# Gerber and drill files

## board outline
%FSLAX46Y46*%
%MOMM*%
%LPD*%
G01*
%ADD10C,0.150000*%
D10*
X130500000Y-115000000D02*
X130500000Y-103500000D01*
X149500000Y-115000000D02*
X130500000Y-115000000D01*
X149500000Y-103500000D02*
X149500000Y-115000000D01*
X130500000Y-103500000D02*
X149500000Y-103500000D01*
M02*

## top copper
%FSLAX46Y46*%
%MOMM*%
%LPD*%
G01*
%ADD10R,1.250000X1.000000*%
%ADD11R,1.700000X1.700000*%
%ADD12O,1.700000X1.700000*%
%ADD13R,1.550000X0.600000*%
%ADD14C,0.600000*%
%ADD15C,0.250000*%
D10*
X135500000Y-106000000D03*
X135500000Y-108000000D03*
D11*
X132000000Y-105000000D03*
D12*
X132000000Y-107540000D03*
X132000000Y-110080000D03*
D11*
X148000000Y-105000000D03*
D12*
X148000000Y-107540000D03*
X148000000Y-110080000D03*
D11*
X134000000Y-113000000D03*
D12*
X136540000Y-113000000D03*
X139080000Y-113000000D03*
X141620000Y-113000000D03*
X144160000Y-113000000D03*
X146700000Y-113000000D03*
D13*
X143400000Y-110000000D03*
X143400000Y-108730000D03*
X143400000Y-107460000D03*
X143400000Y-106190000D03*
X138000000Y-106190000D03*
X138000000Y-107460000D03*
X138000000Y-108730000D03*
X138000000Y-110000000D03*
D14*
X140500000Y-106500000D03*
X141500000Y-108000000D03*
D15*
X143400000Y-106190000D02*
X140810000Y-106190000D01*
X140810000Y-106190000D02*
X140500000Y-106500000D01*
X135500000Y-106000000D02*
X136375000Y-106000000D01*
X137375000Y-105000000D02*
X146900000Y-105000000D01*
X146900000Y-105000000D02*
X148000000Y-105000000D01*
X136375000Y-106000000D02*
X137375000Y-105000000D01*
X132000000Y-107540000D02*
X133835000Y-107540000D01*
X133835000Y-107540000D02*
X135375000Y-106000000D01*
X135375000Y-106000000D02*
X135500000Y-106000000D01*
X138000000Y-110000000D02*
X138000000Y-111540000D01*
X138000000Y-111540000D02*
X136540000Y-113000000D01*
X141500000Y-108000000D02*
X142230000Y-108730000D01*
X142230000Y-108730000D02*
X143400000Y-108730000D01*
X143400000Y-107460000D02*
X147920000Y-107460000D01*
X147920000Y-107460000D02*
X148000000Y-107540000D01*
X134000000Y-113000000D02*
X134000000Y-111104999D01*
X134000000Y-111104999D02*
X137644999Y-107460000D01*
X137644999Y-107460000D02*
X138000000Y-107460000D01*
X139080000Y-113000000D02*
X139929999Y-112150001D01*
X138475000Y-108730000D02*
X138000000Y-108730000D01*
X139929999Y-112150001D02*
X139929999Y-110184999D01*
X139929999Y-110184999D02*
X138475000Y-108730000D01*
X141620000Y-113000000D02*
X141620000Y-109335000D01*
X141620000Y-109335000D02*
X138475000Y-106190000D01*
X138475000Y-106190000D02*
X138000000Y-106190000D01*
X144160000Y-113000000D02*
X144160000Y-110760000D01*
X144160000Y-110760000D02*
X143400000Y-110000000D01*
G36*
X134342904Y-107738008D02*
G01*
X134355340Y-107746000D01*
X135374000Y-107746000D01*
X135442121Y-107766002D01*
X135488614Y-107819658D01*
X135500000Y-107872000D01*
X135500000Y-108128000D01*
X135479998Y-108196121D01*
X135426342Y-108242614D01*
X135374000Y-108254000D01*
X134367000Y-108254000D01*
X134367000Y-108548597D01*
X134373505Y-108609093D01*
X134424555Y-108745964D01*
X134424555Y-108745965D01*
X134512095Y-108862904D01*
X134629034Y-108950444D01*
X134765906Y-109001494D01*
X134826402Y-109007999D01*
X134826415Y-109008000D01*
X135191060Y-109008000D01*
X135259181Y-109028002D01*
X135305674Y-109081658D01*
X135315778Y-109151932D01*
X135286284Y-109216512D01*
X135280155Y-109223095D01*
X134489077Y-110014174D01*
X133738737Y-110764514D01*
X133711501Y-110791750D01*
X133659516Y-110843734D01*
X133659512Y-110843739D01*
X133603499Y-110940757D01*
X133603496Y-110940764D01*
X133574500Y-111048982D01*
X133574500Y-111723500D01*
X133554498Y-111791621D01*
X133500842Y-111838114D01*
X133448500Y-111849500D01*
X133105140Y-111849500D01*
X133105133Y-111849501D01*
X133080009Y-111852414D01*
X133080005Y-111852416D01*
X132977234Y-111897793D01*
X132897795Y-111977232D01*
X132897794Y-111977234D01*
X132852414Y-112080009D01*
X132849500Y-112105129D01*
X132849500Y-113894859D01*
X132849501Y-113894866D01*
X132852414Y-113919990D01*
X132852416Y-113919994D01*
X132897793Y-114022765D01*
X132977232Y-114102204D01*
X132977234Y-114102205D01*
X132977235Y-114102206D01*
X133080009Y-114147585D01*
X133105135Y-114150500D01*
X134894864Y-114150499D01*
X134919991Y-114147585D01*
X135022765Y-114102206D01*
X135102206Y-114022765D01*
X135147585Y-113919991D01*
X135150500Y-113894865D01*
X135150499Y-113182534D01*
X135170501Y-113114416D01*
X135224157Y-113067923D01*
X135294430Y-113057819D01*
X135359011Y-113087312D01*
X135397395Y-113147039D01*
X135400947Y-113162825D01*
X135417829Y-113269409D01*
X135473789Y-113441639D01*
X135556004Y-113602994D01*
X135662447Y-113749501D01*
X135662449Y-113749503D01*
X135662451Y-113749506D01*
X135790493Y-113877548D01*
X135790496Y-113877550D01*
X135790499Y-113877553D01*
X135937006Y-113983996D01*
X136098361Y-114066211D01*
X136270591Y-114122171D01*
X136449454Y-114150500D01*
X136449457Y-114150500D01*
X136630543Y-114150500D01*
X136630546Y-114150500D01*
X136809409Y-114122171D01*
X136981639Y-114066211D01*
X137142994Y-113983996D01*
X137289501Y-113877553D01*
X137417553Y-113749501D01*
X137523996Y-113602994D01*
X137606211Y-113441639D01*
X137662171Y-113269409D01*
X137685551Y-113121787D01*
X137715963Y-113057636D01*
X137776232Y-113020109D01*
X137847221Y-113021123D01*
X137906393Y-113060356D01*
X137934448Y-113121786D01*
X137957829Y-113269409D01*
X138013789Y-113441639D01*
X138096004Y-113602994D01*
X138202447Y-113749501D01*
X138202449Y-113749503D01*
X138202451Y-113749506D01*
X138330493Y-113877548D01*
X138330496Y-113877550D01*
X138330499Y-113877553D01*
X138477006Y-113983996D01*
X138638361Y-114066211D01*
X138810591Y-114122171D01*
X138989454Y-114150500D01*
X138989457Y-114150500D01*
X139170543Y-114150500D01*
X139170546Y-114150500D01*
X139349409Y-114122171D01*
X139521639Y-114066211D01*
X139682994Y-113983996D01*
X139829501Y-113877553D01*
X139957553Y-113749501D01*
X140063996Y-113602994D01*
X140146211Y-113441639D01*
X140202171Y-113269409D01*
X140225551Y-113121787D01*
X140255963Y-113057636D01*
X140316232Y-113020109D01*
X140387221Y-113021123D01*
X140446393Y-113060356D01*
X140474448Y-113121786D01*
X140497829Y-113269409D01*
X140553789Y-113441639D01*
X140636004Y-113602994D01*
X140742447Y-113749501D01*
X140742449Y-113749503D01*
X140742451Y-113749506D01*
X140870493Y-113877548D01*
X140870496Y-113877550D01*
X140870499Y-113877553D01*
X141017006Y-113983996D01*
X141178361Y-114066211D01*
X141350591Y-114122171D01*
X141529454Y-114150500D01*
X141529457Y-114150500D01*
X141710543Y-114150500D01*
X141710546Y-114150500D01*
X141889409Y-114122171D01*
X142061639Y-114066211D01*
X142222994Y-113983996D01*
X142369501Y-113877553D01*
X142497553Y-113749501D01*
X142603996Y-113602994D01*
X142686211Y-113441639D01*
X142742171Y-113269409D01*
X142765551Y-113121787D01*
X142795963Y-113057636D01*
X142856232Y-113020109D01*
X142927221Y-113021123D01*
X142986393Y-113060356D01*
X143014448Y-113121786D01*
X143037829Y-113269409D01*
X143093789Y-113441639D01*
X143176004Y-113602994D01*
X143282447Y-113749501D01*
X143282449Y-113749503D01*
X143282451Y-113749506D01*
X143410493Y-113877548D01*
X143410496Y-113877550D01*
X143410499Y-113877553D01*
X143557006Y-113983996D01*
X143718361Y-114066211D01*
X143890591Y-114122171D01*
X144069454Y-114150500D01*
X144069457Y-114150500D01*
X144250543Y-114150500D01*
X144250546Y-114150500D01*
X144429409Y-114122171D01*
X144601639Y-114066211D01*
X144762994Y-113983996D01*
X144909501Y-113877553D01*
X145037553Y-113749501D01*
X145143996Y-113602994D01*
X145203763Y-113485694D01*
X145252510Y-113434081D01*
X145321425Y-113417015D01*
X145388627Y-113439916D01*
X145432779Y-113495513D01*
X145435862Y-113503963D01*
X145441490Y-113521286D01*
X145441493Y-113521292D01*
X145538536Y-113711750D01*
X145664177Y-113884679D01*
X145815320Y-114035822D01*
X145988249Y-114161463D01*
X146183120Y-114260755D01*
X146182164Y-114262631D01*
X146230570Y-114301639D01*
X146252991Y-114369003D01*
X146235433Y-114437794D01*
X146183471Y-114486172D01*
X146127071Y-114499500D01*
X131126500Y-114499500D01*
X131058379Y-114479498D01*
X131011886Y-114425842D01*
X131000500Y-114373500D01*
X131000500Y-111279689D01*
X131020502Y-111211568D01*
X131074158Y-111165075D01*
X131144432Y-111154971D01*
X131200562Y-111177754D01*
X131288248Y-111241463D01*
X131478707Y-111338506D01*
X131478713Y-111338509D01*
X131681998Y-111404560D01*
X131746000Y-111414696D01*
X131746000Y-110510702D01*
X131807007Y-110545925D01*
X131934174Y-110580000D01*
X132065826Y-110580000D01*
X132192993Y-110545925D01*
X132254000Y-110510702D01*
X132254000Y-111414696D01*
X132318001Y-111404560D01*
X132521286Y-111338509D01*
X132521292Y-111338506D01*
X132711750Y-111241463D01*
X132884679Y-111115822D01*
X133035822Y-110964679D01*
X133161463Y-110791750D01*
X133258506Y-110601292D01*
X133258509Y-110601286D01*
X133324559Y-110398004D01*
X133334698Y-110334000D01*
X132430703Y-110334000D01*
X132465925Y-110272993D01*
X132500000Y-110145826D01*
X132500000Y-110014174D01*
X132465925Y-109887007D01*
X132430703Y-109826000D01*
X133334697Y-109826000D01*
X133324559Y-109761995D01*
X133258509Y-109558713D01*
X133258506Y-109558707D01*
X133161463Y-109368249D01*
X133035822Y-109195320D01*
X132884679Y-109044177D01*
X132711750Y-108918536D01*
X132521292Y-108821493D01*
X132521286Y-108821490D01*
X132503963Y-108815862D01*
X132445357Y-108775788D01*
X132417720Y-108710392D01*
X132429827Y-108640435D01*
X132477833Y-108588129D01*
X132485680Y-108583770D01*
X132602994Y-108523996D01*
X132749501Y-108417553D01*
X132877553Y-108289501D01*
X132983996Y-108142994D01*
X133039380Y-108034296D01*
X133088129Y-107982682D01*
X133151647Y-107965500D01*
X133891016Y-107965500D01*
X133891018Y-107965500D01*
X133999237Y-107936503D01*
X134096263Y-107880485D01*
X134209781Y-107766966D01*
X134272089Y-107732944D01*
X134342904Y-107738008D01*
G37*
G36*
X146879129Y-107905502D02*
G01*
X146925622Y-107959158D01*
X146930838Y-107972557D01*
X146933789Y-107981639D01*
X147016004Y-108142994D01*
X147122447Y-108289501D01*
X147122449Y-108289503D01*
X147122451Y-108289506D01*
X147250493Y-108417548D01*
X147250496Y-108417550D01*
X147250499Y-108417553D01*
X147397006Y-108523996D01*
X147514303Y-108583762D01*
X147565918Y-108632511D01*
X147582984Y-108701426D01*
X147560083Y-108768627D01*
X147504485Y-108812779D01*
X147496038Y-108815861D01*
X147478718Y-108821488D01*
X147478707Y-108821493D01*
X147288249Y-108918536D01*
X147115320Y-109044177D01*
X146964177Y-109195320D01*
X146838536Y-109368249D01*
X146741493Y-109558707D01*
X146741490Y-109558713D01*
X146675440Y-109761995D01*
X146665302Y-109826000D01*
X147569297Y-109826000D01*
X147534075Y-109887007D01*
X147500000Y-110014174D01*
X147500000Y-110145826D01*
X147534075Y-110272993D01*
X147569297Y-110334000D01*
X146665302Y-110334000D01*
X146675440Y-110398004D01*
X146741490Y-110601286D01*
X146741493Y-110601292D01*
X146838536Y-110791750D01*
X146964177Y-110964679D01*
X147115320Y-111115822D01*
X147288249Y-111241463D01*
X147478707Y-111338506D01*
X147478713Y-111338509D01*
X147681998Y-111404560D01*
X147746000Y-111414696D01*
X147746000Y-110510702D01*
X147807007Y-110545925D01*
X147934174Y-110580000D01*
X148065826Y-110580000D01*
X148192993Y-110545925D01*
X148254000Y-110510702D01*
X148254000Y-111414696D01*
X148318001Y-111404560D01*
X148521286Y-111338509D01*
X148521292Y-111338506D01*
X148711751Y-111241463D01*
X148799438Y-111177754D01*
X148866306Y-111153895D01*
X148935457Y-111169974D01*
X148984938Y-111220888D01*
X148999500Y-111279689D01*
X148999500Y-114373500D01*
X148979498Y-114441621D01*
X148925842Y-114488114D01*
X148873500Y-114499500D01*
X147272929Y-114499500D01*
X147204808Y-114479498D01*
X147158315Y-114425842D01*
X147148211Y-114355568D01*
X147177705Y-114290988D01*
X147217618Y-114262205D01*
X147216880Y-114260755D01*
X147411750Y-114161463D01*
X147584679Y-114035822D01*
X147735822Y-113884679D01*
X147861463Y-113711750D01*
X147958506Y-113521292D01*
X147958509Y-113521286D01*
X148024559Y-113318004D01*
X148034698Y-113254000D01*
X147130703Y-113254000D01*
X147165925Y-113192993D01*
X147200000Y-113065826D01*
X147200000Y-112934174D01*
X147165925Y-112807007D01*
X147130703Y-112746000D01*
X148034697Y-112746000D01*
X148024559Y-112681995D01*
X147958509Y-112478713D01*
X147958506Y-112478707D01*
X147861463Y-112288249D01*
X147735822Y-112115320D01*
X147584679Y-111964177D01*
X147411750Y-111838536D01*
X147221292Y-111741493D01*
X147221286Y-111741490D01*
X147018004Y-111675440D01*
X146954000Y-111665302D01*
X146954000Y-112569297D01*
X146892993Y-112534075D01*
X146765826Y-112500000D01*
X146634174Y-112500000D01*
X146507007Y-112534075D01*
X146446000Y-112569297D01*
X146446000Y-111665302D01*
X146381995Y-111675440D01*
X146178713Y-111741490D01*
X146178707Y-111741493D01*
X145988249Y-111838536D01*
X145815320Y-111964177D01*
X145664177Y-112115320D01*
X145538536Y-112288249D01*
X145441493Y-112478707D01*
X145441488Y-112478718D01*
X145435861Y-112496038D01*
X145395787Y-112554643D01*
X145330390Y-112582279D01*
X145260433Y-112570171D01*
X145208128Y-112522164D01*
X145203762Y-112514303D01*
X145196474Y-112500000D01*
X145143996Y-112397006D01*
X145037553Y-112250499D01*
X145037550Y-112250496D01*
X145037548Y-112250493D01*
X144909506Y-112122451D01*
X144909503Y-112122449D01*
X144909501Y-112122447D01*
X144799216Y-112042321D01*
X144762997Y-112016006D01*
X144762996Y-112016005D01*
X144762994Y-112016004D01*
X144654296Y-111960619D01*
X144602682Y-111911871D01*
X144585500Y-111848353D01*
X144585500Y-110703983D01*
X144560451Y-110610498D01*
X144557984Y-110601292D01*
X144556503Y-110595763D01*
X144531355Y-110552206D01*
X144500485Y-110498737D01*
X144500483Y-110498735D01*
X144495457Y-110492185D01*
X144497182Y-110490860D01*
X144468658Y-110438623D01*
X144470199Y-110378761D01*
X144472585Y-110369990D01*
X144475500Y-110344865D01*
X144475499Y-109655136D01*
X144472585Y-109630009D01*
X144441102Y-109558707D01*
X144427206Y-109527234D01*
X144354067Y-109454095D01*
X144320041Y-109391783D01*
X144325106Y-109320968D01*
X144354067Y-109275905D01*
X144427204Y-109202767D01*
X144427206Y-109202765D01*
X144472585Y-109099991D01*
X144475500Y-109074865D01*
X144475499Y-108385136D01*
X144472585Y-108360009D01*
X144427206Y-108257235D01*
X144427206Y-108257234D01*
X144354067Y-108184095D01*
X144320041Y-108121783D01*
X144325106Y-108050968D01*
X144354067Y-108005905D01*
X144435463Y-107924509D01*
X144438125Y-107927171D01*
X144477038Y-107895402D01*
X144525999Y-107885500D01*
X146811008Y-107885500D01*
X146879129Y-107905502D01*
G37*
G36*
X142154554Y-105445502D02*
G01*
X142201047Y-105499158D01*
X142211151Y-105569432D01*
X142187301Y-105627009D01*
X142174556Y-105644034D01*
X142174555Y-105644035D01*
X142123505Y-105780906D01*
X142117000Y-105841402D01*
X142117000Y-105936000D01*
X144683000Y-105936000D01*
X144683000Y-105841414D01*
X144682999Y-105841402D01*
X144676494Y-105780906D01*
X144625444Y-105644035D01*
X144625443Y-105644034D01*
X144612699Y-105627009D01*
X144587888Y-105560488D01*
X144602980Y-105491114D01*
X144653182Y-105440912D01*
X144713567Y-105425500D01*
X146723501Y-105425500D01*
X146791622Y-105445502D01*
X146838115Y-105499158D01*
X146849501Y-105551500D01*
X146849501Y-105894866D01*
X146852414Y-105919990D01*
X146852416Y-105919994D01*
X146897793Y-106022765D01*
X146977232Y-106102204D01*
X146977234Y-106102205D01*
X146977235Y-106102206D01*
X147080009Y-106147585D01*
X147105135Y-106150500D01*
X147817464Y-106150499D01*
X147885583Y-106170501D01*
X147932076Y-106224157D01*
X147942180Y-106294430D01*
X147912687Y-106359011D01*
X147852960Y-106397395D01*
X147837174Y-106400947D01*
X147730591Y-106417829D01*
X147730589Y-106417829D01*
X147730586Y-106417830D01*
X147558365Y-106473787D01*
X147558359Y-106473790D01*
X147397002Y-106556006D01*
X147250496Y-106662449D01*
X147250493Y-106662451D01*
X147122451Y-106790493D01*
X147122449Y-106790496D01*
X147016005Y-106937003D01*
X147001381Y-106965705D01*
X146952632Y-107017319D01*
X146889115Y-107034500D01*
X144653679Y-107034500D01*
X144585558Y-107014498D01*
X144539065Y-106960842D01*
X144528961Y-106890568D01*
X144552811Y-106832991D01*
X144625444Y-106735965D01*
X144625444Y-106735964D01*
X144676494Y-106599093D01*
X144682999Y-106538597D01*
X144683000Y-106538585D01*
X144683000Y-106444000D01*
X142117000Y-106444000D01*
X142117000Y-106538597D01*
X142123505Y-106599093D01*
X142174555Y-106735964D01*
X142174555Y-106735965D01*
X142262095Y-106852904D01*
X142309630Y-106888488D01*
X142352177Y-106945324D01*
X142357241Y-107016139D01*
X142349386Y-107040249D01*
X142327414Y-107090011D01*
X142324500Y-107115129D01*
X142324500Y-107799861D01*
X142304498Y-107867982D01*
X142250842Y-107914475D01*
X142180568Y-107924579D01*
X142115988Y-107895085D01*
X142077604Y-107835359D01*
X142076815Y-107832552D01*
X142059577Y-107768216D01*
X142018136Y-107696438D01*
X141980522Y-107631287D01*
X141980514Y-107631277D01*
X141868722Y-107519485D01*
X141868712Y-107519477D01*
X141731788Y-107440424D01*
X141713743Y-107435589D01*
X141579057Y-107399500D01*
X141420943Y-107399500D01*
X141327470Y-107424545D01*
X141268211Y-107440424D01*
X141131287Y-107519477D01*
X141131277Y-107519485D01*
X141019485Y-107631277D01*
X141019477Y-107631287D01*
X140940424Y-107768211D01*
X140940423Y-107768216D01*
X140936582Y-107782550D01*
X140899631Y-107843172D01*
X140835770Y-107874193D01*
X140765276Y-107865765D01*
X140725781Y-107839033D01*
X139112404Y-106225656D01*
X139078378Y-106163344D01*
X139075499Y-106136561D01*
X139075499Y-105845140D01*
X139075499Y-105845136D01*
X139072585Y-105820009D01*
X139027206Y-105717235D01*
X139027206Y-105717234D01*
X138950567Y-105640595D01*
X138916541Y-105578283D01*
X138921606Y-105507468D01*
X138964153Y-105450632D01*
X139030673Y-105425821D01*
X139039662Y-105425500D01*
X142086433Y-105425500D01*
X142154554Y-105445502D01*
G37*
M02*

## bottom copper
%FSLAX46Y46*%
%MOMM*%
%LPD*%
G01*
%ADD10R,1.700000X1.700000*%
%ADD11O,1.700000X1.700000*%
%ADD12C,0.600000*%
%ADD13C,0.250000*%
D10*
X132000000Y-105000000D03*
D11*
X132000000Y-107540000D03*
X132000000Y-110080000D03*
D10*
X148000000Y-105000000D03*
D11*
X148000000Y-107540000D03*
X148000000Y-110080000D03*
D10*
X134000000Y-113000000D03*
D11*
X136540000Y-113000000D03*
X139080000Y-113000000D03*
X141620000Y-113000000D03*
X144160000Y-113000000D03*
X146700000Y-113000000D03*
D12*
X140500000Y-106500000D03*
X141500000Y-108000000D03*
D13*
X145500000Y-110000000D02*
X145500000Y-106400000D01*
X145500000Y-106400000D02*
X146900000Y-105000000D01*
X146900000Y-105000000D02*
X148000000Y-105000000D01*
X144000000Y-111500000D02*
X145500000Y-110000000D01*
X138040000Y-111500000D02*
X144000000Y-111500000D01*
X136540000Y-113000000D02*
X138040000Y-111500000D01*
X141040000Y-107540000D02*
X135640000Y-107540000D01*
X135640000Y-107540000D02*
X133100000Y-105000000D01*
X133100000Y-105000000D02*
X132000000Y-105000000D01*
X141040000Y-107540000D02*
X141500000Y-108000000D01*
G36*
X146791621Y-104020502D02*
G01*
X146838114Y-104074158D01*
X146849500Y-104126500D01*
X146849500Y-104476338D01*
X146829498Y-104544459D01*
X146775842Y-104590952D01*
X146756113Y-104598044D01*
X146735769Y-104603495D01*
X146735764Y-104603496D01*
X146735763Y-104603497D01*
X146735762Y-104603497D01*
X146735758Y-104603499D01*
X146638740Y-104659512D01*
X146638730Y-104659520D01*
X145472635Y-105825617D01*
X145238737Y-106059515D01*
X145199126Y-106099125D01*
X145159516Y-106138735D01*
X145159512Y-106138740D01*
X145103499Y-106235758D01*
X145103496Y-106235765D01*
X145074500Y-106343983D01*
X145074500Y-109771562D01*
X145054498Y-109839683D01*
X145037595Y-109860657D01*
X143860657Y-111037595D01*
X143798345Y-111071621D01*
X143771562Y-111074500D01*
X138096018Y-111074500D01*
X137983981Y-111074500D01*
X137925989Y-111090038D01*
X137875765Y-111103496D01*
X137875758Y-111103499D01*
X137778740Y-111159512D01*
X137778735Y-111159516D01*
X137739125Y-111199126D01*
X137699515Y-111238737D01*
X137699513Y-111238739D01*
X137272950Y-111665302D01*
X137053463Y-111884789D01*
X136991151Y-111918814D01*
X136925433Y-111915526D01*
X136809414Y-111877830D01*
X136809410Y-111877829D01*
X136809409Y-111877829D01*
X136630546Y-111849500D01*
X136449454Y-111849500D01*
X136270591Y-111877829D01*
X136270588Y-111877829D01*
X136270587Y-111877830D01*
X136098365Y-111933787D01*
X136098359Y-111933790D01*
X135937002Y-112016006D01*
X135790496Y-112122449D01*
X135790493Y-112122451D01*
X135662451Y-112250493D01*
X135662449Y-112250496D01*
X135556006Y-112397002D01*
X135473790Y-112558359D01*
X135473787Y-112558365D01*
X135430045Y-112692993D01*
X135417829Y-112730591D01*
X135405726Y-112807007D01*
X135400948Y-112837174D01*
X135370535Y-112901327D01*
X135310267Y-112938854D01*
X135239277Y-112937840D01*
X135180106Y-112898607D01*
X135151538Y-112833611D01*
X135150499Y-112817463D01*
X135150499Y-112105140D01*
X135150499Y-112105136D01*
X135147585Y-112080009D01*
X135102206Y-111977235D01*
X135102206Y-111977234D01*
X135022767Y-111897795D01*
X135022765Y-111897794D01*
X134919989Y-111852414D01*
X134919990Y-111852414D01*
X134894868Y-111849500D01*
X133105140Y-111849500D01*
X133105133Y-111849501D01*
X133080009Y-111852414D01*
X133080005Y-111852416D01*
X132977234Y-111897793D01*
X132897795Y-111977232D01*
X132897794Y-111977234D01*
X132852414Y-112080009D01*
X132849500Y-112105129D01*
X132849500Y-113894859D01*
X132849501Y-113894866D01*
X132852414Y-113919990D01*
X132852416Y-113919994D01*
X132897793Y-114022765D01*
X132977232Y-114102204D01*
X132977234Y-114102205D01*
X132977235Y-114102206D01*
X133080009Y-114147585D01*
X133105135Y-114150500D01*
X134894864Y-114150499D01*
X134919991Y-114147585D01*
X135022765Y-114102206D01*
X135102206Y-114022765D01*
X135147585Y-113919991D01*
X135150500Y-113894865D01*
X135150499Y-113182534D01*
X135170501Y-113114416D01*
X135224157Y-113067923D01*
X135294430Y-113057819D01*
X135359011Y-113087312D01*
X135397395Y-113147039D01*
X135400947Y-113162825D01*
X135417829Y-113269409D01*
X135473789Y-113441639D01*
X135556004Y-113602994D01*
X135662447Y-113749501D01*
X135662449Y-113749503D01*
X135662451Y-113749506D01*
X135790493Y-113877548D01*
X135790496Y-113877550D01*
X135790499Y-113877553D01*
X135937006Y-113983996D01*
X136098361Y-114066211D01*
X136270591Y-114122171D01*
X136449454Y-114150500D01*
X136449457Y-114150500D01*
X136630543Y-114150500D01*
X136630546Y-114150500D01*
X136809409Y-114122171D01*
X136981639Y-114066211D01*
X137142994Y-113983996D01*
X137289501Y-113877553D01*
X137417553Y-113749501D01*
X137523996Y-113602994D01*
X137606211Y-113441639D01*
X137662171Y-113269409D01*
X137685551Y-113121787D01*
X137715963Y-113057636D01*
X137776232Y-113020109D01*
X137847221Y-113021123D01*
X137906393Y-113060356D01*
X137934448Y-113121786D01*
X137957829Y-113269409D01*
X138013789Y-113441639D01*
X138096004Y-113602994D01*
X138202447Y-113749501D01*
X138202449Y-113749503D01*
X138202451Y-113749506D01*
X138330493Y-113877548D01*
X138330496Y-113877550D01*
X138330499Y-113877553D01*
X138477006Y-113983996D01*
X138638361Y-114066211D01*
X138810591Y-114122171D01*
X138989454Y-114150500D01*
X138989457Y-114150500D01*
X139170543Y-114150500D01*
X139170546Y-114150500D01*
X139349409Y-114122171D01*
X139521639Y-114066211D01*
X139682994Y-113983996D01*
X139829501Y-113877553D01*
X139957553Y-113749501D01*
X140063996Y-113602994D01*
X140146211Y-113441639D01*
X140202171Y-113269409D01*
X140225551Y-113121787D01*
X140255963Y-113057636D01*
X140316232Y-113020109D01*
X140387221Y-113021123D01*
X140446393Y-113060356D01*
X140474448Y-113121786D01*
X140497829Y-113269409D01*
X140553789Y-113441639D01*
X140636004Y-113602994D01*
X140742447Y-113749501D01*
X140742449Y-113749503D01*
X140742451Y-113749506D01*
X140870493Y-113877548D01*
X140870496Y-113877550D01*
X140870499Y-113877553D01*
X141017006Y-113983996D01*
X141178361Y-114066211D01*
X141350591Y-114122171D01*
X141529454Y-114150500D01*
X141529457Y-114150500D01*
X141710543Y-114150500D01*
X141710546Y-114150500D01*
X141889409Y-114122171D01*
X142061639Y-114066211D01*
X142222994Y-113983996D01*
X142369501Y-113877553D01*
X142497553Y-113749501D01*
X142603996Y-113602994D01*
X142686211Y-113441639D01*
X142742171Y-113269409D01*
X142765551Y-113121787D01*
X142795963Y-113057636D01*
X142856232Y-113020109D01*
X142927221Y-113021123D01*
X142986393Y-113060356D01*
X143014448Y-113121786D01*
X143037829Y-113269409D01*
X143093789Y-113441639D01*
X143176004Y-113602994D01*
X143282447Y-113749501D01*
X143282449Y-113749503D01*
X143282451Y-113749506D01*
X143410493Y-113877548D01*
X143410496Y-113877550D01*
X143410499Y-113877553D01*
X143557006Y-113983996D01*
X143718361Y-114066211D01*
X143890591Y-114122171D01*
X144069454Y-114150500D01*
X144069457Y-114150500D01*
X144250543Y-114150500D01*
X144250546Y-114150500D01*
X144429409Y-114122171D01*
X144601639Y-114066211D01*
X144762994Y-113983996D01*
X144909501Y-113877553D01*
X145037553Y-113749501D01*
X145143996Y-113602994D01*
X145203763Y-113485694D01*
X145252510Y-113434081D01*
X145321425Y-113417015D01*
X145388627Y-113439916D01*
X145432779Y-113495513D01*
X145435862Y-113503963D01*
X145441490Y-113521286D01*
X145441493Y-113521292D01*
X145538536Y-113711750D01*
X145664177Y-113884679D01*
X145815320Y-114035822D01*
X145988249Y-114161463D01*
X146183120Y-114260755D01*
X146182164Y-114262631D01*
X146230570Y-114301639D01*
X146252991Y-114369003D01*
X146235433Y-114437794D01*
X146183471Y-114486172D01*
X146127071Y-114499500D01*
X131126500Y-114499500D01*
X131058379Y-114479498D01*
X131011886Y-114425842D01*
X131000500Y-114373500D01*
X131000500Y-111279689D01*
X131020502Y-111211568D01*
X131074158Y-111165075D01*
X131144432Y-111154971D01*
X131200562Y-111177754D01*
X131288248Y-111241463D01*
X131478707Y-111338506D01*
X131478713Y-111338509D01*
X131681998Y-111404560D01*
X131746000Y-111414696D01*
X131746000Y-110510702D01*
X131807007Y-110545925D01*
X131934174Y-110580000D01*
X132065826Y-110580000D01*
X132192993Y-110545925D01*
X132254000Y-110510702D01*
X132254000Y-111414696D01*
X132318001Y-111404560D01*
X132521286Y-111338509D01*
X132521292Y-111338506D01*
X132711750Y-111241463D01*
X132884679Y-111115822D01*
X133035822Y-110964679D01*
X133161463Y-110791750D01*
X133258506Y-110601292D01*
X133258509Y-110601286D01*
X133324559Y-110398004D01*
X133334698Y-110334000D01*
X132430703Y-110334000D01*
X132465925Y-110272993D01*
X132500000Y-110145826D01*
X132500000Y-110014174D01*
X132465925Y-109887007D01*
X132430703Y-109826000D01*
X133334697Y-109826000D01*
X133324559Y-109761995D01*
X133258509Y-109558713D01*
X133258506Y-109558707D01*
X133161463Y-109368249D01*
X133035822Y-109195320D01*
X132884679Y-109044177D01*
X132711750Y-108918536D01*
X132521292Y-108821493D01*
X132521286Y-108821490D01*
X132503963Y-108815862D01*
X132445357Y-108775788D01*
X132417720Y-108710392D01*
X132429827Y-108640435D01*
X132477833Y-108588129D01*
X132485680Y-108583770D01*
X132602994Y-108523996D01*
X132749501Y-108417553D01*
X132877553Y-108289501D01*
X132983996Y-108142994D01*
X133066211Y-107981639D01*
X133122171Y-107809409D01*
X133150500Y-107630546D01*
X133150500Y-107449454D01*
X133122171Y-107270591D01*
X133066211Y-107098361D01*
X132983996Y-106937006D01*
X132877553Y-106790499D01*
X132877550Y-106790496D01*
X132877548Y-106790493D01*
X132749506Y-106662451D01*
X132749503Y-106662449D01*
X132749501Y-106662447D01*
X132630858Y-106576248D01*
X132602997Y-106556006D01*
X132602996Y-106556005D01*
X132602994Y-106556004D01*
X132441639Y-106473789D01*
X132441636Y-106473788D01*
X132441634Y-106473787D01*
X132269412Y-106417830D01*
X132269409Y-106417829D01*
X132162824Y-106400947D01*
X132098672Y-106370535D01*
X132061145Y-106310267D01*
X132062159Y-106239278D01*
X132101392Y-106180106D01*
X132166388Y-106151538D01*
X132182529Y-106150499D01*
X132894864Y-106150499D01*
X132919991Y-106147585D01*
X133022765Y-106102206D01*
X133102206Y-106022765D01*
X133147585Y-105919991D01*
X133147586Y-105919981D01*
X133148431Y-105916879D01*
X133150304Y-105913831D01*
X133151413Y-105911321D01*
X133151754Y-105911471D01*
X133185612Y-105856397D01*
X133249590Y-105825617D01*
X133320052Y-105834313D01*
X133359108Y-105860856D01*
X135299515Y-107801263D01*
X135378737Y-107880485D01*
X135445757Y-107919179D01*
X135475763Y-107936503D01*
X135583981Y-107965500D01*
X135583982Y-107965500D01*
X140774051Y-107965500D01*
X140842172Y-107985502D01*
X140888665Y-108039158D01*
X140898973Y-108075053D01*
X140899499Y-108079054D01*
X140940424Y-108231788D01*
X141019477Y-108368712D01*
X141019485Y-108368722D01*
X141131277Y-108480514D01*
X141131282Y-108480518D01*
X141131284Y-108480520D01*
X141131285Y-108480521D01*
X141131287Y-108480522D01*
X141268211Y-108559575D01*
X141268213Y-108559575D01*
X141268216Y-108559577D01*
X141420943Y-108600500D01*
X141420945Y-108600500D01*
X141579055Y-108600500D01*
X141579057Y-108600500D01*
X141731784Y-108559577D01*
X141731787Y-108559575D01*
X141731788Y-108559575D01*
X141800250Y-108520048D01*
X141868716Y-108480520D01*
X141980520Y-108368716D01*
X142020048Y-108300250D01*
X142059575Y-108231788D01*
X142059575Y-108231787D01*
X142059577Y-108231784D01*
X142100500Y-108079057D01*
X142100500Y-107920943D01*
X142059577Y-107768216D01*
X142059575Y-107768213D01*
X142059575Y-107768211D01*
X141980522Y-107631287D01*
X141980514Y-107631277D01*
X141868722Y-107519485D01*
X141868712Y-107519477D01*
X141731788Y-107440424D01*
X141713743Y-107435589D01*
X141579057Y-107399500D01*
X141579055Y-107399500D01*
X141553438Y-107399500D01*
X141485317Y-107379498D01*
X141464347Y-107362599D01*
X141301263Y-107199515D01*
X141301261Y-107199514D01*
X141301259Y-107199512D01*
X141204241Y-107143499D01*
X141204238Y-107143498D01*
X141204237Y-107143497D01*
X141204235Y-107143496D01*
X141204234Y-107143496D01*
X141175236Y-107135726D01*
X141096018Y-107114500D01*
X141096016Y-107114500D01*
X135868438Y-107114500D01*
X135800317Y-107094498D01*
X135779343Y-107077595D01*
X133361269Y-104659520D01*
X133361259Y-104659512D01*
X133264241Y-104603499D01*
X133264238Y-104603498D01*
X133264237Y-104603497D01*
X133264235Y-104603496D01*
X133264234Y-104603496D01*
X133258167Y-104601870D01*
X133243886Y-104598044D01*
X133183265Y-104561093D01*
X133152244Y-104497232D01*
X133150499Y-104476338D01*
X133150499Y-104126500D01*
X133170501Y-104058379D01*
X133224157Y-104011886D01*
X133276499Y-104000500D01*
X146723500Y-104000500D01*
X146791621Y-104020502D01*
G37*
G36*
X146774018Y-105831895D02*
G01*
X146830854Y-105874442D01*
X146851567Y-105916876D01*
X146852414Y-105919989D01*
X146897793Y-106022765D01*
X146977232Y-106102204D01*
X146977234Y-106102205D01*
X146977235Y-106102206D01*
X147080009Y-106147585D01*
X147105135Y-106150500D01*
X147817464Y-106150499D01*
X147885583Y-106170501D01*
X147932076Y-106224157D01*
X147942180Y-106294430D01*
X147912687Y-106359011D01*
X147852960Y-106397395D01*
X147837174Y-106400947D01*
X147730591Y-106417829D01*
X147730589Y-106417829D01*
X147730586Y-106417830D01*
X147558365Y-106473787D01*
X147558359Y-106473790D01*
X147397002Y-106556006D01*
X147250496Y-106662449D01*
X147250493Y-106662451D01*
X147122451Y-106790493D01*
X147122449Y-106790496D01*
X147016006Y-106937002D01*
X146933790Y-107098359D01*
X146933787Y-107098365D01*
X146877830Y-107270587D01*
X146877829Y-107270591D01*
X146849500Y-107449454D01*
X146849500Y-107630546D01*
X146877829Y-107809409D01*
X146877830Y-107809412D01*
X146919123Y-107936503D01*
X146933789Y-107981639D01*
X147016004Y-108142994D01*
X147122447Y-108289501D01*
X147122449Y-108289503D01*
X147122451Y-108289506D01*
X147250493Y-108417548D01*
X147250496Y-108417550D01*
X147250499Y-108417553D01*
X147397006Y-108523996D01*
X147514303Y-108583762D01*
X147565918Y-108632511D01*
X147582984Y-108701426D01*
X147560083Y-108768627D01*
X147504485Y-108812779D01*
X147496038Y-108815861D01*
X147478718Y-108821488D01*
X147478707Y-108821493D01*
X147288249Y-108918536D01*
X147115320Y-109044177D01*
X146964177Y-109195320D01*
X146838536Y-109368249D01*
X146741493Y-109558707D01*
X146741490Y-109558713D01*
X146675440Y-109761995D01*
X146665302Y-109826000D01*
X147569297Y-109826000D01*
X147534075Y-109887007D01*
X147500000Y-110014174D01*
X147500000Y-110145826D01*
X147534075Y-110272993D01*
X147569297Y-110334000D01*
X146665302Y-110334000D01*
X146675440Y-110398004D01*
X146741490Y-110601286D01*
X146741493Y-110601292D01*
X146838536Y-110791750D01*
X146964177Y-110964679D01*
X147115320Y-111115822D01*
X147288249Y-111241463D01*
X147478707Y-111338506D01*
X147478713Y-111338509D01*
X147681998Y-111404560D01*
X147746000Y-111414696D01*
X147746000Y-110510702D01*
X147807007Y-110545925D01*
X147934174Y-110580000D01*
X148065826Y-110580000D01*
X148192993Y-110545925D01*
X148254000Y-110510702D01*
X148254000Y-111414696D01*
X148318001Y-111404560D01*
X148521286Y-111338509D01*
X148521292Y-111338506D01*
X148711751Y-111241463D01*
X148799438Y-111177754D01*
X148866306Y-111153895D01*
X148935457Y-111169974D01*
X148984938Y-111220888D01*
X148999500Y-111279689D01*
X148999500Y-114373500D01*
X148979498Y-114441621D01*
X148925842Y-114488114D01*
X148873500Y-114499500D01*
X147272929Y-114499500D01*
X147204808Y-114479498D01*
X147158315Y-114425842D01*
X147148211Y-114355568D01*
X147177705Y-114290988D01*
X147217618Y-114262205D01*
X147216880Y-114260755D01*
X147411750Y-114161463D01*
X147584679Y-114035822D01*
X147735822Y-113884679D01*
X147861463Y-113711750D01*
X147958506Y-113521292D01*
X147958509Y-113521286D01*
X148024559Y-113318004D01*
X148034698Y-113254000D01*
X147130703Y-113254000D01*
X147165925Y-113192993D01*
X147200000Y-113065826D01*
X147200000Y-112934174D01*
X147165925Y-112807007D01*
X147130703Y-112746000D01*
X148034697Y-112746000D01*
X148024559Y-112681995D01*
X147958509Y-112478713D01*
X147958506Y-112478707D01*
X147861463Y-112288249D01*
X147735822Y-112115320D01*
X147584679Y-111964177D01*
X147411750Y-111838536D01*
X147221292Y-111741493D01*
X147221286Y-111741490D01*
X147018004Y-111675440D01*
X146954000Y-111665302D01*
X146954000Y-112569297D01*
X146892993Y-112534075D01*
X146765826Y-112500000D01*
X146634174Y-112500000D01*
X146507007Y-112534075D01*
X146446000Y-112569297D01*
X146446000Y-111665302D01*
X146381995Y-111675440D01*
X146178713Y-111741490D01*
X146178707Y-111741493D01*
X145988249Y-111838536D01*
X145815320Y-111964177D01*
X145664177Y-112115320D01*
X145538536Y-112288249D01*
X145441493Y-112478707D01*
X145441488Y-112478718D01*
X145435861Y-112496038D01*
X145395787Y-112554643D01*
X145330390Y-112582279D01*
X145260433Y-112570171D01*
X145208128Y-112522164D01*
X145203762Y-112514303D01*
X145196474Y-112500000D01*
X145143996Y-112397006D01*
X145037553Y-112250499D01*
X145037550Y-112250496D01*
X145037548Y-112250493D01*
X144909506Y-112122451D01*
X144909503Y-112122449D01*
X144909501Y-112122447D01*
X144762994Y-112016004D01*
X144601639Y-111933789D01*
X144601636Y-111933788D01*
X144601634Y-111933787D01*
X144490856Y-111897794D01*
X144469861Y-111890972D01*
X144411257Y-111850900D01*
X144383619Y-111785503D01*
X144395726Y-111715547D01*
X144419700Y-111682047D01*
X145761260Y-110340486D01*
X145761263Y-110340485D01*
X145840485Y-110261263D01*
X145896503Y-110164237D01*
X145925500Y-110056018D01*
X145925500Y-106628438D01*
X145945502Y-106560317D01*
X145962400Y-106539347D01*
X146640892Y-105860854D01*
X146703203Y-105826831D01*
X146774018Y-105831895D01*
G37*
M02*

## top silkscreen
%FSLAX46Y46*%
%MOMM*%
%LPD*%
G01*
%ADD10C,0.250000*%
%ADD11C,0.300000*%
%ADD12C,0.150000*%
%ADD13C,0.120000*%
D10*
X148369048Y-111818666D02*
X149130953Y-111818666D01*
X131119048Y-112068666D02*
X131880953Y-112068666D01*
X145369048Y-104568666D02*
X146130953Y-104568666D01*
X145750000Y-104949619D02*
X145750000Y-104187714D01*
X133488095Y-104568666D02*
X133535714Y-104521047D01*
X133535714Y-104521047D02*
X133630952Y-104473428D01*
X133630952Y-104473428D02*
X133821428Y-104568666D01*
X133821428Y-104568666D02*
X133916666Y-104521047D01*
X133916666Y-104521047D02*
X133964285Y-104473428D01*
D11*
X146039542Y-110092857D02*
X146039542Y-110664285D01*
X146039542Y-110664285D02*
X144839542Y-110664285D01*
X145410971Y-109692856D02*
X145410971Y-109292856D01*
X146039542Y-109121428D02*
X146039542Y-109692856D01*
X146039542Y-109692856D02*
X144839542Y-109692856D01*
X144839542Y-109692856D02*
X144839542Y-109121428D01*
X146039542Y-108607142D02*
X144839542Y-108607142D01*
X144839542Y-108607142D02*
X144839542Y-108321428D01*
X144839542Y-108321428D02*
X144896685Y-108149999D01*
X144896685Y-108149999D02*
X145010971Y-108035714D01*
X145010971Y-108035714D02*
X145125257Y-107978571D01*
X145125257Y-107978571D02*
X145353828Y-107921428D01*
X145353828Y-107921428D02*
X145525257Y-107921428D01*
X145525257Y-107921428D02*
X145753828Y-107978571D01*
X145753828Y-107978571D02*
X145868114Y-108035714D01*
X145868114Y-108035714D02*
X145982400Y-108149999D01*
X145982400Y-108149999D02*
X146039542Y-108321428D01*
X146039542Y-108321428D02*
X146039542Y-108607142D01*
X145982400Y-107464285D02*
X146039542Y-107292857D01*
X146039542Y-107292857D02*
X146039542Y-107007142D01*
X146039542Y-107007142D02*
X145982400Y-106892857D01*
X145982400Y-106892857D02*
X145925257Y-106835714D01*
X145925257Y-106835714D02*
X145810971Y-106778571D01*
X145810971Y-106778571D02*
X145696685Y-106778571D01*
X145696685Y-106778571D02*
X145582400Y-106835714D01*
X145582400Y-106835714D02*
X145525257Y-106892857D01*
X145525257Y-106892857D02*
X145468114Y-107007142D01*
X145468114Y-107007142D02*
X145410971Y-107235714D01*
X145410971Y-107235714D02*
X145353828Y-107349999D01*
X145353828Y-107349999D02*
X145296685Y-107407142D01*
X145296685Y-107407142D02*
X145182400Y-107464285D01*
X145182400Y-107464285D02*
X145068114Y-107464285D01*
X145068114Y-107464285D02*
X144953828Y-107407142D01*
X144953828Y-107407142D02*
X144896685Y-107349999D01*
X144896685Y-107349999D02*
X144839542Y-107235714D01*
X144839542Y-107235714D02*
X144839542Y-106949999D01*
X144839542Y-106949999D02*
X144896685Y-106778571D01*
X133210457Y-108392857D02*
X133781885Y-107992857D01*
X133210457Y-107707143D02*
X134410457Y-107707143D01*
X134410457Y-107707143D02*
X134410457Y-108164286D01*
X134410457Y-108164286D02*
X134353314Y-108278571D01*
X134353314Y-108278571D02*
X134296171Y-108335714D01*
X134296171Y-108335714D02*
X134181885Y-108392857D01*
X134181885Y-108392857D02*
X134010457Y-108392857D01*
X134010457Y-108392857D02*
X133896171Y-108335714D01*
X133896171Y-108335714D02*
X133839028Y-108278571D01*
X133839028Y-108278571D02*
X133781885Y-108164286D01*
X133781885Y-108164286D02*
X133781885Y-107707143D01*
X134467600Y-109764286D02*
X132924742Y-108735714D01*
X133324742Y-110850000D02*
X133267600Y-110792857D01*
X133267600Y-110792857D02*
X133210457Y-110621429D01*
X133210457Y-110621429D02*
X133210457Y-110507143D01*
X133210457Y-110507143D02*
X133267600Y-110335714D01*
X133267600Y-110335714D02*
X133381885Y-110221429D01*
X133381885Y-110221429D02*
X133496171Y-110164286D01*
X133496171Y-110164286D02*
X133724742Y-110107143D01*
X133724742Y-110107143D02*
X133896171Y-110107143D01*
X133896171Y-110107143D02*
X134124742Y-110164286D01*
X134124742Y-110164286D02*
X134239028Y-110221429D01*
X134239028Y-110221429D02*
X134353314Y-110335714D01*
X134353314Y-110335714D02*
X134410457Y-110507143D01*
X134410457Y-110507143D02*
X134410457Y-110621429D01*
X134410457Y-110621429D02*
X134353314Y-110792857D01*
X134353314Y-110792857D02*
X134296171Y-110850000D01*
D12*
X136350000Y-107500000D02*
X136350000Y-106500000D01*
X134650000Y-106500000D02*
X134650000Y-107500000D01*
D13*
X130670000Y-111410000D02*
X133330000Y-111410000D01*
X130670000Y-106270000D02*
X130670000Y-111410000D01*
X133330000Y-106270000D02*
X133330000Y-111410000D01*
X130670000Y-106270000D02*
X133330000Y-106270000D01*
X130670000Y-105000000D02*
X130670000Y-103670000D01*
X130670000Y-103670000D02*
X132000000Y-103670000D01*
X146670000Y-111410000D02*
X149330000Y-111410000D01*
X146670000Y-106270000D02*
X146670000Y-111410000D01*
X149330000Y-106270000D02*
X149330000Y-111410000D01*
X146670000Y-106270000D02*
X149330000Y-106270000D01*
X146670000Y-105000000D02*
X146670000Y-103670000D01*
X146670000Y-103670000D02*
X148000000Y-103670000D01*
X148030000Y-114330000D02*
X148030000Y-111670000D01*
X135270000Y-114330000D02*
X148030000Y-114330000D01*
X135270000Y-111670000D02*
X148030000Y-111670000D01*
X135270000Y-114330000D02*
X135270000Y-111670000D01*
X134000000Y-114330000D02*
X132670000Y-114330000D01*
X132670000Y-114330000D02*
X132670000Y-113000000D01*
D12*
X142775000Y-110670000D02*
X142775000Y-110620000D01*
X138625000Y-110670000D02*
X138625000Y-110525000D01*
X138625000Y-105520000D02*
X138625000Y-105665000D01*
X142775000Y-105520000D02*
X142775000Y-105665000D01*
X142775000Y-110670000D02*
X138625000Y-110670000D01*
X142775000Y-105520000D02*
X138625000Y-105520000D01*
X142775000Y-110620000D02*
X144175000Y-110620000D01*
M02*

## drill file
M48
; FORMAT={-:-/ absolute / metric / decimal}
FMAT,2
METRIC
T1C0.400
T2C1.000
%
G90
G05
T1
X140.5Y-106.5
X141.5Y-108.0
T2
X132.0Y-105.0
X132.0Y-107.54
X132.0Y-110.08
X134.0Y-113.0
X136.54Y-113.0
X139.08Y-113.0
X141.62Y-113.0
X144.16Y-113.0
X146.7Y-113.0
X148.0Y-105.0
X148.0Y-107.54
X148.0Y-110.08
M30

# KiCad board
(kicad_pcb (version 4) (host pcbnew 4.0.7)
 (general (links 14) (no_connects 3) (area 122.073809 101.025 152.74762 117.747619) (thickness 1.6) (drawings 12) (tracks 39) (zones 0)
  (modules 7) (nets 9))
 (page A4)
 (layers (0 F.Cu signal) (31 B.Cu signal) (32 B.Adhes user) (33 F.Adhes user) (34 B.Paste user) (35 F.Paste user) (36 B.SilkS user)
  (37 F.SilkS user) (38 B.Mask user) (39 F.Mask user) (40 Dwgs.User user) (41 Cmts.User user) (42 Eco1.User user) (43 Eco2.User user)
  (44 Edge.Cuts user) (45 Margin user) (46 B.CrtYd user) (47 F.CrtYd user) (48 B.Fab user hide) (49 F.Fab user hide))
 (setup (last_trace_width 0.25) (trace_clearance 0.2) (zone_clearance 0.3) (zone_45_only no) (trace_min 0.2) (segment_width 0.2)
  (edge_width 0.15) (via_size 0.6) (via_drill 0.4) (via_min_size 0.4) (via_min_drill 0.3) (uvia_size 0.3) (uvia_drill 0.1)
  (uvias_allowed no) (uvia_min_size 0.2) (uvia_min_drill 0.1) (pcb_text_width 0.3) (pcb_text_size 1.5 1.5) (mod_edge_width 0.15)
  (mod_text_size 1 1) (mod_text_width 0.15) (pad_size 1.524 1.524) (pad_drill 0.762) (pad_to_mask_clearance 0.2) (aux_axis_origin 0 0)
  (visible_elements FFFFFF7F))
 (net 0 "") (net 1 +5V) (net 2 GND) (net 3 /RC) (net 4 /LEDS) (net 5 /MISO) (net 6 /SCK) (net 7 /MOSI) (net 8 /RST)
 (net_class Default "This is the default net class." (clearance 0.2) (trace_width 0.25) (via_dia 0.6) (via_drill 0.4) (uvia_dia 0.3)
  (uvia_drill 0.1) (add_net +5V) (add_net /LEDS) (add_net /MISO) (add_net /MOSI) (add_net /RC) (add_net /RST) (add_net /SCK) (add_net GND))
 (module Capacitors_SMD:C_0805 (layer F.Cu) (at 135.5 107 270)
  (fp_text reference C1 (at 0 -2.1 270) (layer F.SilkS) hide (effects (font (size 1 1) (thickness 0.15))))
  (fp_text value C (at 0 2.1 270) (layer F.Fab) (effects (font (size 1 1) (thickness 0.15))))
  (fp_line (start 0.5 -0.85) (end -0.5 -0.85) (layer F.SilkS) (width 0.15))
  (fp_line (start -0.5 0.85) (end 0.5 0.85) (layer F.SilkS) (width 0.15))
  (pad 1 smd rect (at -1 0 270) (size 1 1.25) (layers F.Cu F.Paste F.Mask) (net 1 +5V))
  (pad 2 smd rect (at 1 0 270) (size 1 1.25) (layers F.Cu F.Paste F.Mask) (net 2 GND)))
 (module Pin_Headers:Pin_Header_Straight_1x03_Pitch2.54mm (layer F.Cu) (at 132 105)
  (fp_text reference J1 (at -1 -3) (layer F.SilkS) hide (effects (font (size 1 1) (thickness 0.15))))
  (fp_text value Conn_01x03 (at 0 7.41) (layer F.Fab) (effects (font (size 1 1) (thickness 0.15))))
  (fp_line (start -1.33 6.41) (end 1.33 6.41) (layer F.SilkS) (width 0.12))
  (fp_line (start -1.33 1.27) (end -1.33 6.41) (layer F.SilkS) (width 0.12))
  (fp_line (start 1.33 1.27) (end 1.33 6.41) (layer F.SilkS) (width 0.12))
  (fp_line (start -1.33 1.27) (end 1.33 1.27) (layer F.SilkS) (width 0.12))
  (fp_line (start -1.33 0) (end -1.33 -1.33) (layer F.SilkS) (width 0.12))
  (fp_line (start -1.33 -1.33) (end 0 -1.33) (layer F.SilkS) (width 0.12))
  (pad 1 thru_hole rect (at 0 0) (size 1.7 1.7) (drill 1) (layers *.Cu *.Mask) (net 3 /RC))
  (pad 2 thru_hole oval (at 0 2.54) (size 1.7 1.7) (drill 1) (layers *.Cu *.Mask) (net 1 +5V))
  (pad 3 thru_hole oval (at 0 5.08) (size 1.7 1.7) (drill 1) (layers *.Cu *.Mask) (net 2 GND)))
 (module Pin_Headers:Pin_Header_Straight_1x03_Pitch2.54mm (layer F.Cu) (at 148 105)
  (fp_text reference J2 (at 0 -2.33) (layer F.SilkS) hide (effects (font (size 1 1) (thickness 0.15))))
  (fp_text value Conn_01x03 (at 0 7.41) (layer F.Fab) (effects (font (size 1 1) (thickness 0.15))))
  (fp_line (start -1.33 6.41) (end 1.33 6.41) (layer F.SilkS) (width 0.12))
  (fp_line (start -1.33 1.27) (end -1.33 6.41) (layer F.SilkS) (width 0.12))
  (fp_line (start 1.33 1.27) (end 1.33 6.41) (layer F.SilkS) (width 0.12))
  (fp_line (start -1.33 1.27) (end 1.33 1.27) (layer F.SilkS) (width 0.12))
  (fp_line (start -1.33 0) (end -1.33 -1.33) (layer F.SilkS) (width 0.12))
  (fp_line (start -1.33 -1.33) (end 0 -1.33) (layer F.SilkS) (width 0.12))
  (pad 1 thru_hole rect (at 0 0) (size 1.7 1.7) (drill 1) (layers *.Cu *.Mask) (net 1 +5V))
  (pad 2 thru_hole oval (at 0 2.54) (size 1.7 1.7) (drill 1) (layers *.Cu *.Mask) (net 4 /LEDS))
  (pad 3 thru_hole oval (at 0 5.08) (size 1.7 1.7) (drill 1) (layers *.Cu *.Mask) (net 2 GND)))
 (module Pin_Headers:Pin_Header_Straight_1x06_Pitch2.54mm (layer F.Cu) (at 134 113 90)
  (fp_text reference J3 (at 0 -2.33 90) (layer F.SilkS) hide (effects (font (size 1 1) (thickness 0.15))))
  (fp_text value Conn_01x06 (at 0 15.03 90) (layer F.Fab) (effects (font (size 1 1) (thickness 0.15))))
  (fp_line (start -1.33 14.03) (end 1.33 14.03) (layer F.SilkS) (width 0.12))
  (fp_line (start -1.33 1.27) (end -1.33 14.03) (layer F.SilkS) (width 0.12))
  (fp_line (start 1.33 1.27) (end 1.33 14.03) (layer F.SilkS) (width 0.12))
  (fp_line (start -1.33 1.27) (end 1.33 1.27) (layer F.SilkS) (width 0.12))
  (fp_line (start -1.33 0) (end -1.33 -1.33) (layer F.SilkS) (width 0.12))
  (fp_line (start -1.33 -1.33) (end 0 -1.33) (layer F.SilkS) (width 0.12))
  (pad 1 thru_hole rect (at 0 0 90) (size 1.7 1.7) (drill 1) (layers *.Cu *.Mask) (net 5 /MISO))
  (pad 2 thru_hole oval (at 0 2.54 90) (size 1.7 1.7) (drill 1) (layers *.Cu *.Mask) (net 1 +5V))
  (pad 3 thru_hole oval (at 0 5.08 90) (size 1.7 1.7) (drill 1) (layers *.Cu *.Mask) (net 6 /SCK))
  (pad 4 thru_hole oval (at 0 7.62 90) (size 1.7 1.7) (drill 1) (layers *.Cu *.Mask) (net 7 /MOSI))
  (pad 5 thru_hole oval (at 0 10.16 90) (size 1.7 1.7) (drill 1) (layers *.Cu *.Mask) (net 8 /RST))
  (pad 6 thru_hole oval (at 0 12.7 90) (size 1.7 1.7) (drill 1) (layers *.Cu *.Mask) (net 2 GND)))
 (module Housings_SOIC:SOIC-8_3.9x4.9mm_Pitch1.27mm (layer F.Cu) (at 140.7 108.095 180)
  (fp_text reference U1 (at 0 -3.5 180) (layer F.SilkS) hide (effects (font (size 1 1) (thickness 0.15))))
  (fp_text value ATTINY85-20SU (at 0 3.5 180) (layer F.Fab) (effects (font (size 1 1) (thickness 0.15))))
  (fp_line (start -2.075 -2.575) (end -2.075 -2.525) (layer F.SilkS) (width 0.15))
  (fp_line (start 2.075 -2.575) (end 2.075 -2.43) (layer F.SilkS) (width 0.15))
  (fp_line (start 2.075 2.575) (end 2.075 2.43) (layer F.SilkS) (width 0.15))
  (fp_line (start -2.075 2.575) (end -2.075 2.43) (layer F.SilkS) (width 0.15))
  (fp_line (start -2.075 -2.575) (end 2.075 -2.575) (layer F.SilkS) (width 0.15))
  (fp_line (start -2.075 2.575) (end 2.075 2.575) (layer F.SilkS) (width 0.15))
  (fp_line (start -2.075 -2.525) (end -3.475 -2.525) (layer F.SilkS) (width 0.15))
  (pad 1 smd rect (at -2.7 -1.905 180) (size 1.55 0.6) (layers F.Cu F.Paste F.Mask) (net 8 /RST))
  (pad 2 smd rect (at -2.7 -0.635 180) (size 1.55 0.6) (layers F.Cu F.Paste F.Mask) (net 3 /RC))
  (pad 3 smd rect (at -2.7 0.635 180) (size 1.55 0.6) (layers F.Cu F.Paste F.Mask) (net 4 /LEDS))
  (pad 4 smd rect (at -2.7 1.905 180) (size 1.55 0.6) (layers F.Cu F.Paste F.Mask) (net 2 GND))
  (pad 5 smd rect (at 2.7 1.905 180) (size 1.55 0.6) (layers F.Cu F.Paste F.Mask) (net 7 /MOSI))
  (pad 6 smd rect (at 2.7 0.635 180) (size 1.55 0.6) (layers F.Cu F.Paste F.Mask) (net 5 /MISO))
  (pad 7 smd rect (at 2.7 -0.635 180) (size 1.55 0.6) (layers F.Cu F.Paste F.Mask) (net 6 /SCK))
  (pad 8 smd rect (at 2.7 -1.905 180) (size 1.55 0.6) (layers F.Cu F.Paste F.Mask) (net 1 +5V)))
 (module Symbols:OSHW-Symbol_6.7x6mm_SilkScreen (layer B.Cu) (at 136.5 108.75 180)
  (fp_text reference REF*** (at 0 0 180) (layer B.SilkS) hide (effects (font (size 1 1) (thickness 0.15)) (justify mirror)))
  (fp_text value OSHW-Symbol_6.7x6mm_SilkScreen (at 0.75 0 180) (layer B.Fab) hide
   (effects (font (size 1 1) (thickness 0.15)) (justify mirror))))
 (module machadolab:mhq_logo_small (layer B.Cu) (at 143.25 109 180)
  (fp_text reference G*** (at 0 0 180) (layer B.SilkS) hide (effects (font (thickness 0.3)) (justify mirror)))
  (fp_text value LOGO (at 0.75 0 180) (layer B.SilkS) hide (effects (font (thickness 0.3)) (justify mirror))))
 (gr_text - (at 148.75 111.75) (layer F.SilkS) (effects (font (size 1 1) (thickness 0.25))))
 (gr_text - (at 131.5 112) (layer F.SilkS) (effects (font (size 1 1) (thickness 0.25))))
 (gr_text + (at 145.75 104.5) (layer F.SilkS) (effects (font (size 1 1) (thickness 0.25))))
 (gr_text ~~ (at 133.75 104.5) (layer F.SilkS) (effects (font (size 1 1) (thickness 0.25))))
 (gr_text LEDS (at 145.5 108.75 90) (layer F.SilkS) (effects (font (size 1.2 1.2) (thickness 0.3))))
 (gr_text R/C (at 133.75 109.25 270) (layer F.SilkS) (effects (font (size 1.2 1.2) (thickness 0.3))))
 (gr_line (start 130.5 115) (end 130.5 103.5) (layer Edge.Cuts) (width 0.15))
 (gr_line (start 149.5 115) (end 130.5 115) (layer Edge.Cuts) (width 0.15))
 (gr_line (start 149.5 103.5) (end 149.5 115) (layer Edge.Cuts) (width 0.15))
 (gr_line (start 130.5 103.5) (end 149.5 103.5) (layer Edge.Cuts) (width 0.15))
 (segment (start 143.4 106.19) (end 140.81 106.19) (width 0.25) (layer F.Cu) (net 2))
 (segment (start 140.81 106.19) (end 140.5 106.5) (width 0.25) (layer F.Cu) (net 2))
 (via (at 140.5 106.5) (size 0.6) (drill 0.4) (layers F.Cu B.Cu) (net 2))
 (segment (start 135.5 106) (end 136.375 106) (width 0.25) (layer F.Cu) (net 1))
 (segment (start 137.375 105) (end 146.9 105) (width 0.25) (layer F.Cu) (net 1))
 (segment (start 146.9 105) (end 148 105) (width 0.25) (layer F.Cu) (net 1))
 (segment (start 136.375 106) (end 137.375 105) (width 0.25) (layer F.Cu) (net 1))
 (segment (start 132 107.54) (end 133.835 107.54) (width 0.25) (layer F.Cu) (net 1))
 (segment (start 133.835 107.54) (end 135.375 106) (width 0.25) (layer F.Cu) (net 1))
 (segment (start 135.375 106) (end 135.5 106) (width 0.25) (layer F.Cu) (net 1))
 (segment (start 145.5 110) (end 145.5 106.4) (width 0.25) (layer B.Cu) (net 1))
 (segment (start 145.5 106.4) (end 146.9 105) (width 0.25) (layer B.Cu) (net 1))
 (segment (start 146.9 105) (end 148 105) (width 0.25) (layer B.Cu) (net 1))
 (segment (start 144 111.5) (end 145.5 110) (width 0.25) (layer B.Cu) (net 1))
 (segment (start 138.04 111.5) (end 144 111.5) (width 0.25) (layer B.Cu) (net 1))
 (segment (start 136.54 113) (end 138.04 111.5) (width 0.25) (layer B.Cu) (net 1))
 (segment (start 138 110) (end 138 111.54) (width 0.25) (layer F.Cu) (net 1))
 (segment (start 138 111.54) (end 136.54 113) (width 0.25) (layer F.Cu) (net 1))
 (segment (start 141.04 107.54) (end 135.64 107.54) (width 0.25) (layer B.Cu) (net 3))
 (segment (start 135.64 107.54) (end 133.1 105) (width 0.25) (layer B.Cu) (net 3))
 (segment (start 133.1 105) (end 132 105) (width 0.25) (layer B.Cu) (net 3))
 (segment (start 141.5 108) (end 142.23 108.73) (width 0.25) (layer F.Cu) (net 3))
 (segment (start 142.23 108.73) (end 143.4 108.73) (width 0.25) (layer F.Cu) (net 3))
 (via (at 141.5 108) (size 0.6) (drill 0.4) (layers F.Cu B.Cu) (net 3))
 (segment (start 141.04 107.54) (end 141.5 108) (width 0.25) (layer B.Cu) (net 3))
 (segment (start 143.4 107.46) (end 147.92 107.46) (width 0.25) (layer F.Cu) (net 4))
 (segment (start 147.92 107.46) (end 148 107.54) (width 0.25) (layer F.Cu) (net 4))
 (segment (start 134 113) (end 134 111.104999) (width 0.25) (layer F.Cu) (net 5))
 (segment (start 134 111.104999) (end 137.644999 107.46) (width 0.25) (layer F.Cu) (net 5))
 (segment (start 137.644999 107.46) (end 138 107.46) (width 0.25) (layer F.Cu) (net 5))
 (segment (start 139.08 113) (end 139.929999 112.150001) (width 0.25) (layer F.Cu) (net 6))
 (segment (start 138.475 108.73) (end 138 108.73) (width 0.25) (layer F.Cu) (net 6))
 (segment (start 139.929999 112.150001) (end 139.929999 110.184999) (width 0.25) (layer F.Cu) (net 6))
 (segment (start 139.929999 110.184999) (end 138.475 108.73) (width 0.25) (layer F.Cu) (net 6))
 (segment (start 141.62 113) (end 141.62 109.335) (width 0.25) (layer F.Cu) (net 7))
 (segment (start 141.62 109.335) (end 138.475 106.19) (width 0.25) (layer F.Cu) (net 7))
 (segment (start 138.475 106.19) (end 138 106.19) (width 0.25) (layer F.Cu) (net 7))
 (segment (start 144.16 113) (end 144.16 110.76) (width 0.25) (layer F.Cu) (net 8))
 (segment (start 144.16 110.76) (end 143.4 110) (width 0.25) (layer F.Cu) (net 8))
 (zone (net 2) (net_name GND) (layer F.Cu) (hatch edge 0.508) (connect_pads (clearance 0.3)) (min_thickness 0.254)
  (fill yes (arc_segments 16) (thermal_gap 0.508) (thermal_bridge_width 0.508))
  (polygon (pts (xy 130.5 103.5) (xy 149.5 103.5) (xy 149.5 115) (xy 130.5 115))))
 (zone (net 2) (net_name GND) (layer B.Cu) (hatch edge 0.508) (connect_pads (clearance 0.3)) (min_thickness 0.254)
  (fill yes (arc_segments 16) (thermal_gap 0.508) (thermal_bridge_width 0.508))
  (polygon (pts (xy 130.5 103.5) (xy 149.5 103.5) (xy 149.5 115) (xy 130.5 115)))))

